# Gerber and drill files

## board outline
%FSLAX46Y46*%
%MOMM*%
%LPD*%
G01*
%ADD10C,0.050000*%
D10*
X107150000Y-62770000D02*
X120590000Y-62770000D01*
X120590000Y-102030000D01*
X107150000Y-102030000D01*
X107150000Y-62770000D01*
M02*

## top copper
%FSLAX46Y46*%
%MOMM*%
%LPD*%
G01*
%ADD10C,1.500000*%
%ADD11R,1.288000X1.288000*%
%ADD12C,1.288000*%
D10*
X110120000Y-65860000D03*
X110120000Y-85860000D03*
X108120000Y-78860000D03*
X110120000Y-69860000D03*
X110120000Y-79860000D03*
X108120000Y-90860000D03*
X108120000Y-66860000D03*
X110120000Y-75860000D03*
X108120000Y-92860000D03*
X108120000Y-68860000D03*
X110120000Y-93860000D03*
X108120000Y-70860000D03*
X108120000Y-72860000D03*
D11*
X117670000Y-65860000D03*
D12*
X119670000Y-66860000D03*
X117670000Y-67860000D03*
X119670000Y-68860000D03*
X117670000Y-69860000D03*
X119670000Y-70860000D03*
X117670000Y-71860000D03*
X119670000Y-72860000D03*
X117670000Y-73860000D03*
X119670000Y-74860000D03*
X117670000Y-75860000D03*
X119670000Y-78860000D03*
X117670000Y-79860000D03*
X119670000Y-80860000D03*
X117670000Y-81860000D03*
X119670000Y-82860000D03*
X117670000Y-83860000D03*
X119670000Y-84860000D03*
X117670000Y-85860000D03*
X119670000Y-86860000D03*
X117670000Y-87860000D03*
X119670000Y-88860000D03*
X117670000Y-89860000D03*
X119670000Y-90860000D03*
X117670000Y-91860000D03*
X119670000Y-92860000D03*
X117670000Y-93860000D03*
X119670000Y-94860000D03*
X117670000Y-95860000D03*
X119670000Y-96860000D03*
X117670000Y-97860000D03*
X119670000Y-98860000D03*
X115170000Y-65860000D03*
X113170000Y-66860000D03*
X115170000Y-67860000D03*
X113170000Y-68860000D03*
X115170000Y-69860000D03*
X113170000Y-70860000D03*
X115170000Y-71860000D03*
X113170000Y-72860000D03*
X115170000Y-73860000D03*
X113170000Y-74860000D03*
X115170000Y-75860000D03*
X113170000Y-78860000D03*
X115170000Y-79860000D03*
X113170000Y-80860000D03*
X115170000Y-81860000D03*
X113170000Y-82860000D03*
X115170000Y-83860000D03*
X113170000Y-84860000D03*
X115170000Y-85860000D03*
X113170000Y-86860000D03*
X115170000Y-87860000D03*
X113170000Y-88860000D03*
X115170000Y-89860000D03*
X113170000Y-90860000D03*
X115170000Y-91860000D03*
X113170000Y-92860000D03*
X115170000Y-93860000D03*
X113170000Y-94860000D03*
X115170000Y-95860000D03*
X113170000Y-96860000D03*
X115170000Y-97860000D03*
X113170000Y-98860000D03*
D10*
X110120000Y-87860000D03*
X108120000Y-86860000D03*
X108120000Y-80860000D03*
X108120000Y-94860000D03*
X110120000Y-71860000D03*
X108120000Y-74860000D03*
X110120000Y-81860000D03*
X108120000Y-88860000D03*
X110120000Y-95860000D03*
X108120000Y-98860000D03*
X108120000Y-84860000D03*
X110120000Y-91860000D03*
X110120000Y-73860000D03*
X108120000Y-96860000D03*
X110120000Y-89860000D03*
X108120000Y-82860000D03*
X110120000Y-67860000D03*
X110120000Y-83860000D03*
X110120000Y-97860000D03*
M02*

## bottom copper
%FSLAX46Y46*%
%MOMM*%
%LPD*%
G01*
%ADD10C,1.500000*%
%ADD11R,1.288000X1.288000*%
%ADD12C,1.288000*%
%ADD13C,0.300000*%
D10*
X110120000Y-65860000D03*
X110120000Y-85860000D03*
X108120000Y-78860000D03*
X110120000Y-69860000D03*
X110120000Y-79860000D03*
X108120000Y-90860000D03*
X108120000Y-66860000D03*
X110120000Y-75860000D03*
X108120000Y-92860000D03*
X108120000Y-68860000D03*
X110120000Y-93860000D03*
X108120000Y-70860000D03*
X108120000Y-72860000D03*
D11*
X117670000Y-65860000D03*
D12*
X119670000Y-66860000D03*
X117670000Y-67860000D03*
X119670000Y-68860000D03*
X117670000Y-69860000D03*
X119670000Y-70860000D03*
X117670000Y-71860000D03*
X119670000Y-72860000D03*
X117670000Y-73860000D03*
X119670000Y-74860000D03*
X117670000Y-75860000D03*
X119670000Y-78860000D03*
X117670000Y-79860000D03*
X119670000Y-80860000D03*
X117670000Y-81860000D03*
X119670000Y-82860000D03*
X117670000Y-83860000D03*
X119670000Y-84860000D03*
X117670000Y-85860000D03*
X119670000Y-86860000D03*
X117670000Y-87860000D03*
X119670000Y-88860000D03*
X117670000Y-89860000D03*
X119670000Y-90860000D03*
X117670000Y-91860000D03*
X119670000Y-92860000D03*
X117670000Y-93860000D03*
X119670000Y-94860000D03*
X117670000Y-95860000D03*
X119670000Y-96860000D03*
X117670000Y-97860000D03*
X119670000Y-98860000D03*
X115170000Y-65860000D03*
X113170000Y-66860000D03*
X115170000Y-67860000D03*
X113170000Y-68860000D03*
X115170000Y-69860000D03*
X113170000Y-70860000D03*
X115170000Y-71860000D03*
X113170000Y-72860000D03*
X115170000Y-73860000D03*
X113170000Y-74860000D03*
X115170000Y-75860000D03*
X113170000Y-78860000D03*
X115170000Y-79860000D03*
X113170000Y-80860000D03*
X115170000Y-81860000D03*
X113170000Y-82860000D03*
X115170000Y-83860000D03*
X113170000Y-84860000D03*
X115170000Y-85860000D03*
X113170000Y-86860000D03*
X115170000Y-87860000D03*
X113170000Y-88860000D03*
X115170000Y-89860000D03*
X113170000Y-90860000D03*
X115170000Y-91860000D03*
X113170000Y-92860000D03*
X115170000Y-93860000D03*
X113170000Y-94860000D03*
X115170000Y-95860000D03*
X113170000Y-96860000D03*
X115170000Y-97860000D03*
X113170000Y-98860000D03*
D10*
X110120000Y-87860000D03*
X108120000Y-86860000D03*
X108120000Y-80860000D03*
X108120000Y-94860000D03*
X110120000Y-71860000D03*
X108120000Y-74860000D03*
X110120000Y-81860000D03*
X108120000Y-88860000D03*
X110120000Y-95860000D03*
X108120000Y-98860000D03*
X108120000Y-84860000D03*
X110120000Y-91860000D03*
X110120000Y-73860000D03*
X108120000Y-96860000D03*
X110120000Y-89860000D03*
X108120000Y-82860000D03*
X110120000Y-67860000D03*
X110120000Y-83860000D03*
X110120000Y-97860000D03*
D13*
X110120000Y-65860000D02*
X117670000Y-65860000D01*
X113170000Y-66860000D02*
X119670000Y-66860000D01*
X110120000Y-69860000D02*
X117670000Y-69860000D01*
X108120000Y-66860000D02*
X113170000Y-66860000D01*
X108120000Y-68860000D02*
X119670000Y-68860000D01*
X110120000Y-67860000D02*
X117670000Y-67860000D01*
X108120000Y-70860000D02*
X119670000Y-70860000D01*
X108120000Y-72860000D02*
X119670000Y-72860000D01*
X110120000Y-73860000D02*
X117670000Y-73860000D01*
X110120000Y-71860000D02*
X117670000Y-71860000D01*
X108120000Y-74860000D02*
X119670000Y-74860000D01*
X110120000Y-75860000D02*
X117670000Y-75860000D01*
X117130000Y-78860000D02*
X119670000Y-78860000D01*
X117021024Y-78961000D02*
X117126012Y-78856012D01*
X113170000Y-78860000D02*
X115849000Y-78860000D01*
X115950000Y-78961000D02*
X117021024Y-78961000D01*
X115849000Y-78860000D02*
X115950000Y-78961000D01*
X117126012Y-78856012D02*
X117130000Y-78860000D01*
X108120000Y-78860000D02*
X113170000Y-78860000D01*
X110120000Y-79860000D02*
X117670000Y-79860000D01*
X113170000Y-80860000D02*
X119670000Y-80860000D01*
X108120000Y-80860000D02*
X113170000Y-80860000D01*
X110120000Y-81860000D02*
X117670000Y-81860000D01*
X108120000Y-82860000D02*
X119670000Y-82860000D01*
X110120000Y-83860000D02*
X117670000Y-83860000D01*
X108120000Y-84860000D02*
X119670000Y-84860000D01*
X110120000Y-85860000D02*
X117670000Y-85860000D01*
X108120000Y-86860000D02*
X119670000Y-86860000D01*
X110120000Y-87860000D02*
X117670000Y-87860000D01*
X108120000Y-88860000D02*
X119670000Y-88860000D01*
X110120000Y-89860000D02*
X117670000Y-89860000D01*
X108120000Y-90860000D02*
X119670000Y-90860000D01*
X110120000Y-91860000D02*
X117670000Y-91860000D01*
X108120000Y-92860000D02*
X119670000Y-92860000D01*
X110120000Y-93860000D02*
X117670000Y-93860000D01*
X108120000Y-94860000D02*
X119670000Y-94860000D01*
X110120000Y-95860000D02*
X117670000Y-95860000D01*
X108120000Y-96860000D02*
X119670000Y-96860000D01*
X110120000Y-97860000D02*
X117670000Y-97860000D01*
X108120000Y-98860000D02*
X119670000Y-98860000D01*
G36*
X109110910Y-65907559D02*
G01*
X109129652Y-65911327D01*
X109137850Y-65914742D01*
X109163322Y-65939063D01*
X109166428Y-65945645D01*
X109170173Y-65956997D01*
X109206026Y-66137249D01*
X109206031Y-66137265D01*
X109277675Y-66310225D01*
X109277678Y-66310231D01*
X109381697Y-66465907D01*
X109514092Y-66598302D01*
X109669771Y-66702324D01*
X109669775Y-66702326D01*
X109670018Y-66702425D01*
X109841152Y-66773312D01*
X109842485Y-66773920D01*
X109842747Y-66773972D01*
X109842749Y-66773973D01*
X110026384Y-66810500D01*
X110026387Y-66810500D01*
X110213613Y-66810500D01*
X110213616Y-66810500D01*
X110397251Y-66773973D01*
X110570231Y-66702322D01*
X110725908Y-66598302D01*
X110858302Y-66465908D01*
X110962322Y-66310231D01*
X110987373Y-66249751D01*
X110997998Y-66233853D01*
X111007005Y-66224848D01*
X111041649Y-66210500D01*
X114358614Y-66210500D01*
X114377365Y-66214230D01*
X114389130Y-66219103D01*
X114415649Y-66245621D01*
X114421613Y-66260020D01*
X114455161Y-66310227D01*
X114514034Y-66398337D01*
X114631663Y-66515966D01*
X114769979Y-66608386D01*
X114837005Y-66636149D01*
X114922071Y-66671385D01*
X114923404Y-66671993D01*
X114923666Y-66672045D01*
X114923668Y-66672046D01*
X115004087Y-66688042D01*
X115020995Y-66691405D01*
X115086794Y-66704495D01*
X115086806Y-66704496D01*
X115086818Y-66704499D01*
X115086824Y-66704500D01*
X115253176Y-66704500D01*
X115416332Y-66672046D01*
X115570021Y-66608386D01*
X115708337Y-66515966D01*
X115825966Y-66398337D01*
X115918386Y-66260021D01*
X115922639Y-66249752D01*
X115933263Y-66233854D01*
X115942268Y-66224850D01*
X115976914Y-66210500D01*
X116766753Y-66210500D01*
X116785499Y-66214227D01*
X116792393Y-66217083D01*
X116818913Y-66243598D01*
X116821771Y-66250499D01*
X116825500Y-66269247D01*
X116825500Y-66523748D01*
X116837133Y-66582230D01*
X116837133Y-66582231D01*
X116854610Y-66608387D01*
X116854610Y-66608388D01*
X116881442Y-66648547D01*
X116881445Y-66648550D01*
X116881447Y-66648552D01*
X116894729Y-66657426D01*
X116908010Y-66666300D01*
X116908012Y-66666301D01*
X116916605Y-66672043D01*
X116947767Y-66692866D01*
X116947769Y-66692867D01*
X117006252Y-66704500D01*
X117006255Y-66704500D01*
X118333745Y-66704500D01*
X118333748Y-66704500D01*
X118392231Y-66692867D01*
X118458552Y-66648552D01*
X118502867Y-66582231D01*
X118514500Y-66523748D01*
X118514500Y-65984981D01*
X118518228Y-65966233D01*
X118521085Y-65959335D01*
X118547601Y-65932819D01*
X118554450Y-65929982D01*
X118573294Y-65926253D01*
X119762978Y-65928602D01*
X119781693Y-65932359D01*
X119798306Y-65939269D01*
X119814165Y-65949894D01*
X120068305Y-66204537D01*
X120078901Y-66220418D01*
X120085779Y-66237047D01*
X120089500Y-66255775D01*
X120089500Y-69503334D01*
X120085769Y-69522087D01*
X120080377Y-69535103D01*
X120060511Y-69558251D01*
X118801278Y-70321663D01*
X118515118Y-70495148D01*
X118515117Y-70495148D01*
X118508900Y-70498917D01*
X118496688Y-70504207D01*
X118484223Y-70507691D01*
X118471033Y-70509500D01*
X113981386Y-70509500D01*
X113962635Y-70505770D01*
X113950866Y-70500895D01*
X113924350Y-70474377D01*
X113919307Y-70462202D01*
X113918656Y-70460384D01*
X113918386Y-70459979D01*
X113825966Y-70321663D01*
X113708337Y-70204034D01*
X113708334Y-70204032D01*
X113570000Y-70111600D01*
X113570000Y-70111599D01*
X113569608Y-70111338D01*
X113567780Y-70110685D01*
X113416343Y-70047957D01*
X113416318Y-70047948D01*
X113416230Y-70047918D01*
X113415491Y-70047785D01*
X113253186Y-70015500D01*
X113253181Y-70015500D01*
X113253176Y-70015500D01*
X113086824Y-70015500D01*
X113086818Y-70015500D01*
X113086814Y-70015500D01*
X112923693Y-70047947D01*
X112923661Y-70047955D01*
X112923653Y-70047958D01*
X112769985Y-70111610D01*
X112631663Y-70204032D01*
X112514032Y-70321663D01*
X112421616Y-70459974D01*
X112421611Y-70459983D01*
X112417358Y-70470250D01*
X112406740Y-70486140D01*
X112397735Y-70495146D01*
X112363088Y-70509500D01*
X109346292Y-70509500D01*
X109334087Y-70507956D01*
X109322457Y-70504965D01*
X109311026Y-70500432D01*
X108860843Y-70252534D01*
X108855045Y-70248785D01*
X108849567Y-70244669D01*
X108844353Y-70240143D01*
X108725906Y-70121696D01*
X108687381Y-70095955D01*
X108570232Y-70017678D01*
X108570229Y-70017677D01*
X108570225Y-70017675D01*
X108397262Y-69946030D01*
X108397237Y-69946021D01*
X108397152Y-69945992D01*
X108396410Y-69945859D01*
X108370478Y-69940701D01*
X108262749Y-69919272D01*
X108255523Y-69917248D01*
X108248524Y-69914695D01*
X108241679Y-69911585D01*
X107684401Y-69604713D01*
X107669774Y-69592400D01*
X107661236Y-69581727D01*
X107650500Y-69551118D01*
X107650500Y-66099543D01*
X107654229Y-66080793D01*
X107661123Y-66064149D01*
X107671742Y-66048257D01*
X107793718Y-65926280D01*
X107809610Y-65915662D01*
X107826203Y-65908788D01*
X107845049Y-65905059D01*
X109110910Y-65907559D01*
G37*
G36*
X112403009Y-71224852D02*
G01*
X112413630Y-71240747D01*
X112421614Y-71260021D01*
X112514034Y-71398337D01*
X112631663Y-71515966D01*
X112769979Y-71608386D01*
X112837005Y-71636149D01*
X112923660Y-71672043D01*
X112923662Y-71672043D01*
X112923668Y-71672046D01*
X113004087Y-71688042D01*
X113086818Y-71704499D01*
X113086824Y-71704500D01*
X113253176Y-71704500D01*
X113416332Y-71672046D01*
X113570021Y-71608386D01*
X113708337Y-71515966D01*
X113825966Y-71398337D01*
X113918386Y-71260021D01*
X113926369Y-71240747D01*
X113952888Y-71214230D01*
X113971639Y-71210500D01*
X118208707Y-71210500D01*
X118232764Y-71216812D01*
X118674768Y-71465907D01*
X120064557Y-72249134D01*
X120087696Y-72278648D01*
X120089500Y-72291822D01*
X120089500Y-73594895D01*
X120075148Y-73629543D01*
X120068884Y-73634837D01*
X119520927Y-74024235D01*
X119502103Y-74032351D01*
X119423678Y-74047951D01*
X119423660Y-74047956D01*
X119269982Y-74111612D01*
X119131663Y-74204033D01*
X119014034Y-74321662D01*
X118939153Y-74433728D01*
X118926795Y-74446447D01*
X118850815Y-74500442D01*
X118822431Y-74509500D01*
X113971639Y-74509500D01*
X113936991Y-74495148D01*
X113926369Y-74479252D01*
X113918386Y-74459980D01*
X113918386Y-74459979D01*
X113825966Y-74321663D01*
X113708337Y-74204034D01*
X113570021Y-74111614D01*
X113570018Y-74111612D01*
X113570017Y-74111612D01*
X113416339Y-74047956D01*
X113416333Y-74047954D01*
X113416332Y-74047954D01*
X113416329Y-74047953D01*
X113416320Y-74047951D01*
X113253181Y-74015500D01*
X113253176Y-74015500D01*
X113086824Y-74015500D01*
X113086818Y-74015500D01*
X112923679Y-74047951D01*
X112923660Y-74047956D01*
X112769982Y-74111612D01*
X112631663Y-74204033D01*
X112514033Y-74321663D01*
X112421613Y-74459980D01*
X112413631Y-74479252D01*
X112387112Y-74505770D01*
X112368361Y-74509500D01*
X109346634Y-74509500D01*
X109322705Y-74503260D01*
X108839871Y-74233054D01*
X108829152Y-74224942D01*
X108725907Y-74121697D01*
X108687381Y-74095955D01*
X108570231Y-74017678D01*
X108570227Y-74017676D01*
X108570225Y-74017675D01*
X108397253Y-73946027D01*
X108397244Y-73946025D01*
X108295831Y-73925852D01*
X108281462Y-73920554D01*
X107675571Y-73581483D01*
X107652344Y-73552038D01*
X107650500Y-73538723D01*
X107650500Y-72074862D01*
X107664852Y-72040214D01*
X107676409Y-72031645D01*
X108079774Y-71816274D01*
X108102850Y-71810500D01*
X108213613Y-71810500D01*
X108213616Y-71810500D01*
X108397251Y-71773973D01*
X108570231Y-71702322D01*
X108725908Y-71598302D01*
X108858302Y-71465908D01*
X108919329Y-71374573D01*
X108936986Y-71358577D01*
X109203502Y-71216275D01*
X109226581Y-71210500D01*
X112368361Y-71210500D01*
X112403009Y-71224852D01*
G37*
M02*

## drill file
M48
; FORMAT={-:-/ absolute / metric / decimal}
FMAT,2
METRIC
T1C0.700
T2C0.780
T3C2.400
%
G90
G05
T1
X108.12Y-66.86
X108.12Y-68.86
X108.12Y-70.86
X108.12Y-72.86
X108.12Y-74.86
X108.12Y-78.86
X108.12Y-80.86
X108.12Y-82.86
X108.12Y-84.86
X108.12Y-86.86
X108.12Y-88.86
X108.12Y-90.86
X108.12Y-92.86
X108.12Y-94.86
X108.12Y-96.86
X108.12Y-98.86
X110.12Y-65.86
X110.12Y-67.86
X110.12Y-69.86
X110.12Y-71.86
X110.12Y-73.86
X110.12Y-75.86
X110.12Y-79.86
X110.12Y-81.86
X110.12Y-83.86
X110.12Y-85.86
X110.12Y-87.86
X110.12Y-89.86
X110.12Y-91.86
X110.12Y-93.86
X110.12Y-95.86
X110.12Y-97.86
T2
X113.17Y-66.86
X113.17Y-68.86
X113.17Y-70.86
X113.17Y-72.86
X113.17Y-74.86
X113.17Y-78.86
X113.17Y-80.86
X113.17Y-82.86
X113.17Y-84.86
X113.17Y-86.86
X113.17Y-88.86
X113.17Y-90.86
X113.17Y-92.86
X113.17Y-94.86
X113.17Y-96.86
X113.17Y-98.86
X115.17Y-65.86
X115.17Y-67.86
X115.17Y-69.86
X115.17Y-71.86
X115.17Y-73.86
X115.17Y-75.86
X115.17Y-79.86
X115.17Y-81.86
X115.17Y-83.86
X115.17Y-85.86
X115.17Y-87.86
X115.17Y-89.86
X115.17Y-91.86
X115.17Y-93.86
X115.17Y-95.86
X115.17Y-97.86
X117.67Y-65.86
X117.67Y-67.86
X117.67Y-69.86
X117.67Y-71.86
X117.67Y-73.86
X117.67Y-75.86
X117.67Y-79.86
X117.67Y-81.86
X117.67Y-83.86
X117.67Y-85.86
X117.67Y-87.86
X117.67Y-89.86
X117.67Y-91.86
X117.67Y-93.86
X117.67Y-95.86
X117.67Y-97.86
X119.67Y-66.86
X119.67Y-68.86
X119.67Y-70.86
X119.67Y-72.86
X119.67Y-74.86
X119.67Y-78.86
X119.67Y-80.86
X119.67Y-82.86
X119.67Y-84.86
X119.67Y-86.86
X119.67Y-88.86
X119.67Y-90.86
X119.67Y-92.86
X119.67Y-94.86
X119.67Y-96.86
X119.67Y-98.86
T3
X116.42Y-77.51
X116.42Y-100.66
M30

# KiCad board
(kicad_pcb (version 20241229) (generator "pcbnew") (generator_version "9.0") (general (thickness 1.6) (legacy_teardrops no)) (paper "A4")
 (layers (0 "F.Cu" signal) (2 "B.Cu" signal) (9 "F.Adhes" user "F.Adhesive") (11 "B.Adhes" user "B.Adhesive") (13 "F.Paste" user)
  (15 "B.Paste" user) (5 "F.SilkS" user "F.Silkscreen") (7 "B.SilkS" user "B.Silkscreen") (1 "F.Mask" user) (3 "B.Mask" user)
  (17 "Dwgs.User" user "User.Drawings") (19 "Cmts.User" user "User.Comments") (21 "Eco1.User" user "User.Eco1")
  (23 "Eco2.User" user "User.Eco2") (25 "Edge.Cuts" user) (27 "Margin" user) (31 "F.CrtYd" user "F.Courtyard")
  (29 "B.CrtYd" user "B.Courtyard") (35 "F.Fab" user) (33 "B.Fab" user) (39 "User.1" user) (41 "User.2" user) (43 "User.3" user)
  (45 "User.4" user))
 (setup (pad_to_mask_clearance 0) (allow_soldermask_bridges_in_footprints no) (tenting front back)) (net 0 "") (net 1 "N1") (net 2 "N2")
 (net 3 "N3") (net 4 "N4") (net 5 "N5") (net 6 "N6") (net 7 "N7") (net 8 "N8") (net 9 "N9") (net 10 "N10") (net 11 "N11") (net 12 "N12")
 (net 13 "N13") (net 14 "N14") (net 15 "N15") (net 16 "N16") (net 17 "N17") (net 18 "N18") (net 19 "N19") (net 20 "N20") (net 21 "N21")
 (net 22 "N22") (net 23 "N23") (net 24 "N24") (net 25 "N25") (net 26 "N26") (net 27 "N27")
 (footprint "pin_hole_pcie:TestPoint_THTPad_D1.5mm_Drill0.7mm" (layer "F.Cu") (at 110.12 65.86 180)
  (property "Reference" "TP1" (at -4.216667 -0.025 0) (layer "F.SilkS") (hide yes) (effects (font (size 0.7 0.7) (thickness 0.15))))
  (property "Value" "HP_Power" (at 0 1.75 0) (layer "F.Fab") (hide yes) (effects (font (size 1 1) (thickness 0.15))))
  (pad "1" thru_hole circle (at 0 0 180) (size 1.5 1.5) (drill 0.7) (layers "*.Cu" "*.Mask") (remove_unused_layers no) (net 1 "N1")))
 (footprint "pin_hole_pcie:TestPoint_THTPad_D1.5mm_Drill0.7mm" (layer "F.Cu") (at 110.12 85.86 180)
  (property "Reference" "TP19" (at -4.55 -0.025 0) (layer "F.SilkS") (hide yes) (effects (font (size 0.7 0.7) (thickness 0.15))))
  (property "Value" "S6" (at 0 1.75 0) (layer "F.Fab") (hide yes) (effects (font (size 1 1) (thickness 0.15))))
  (pad "1" thru_hole circle (at 0 0 180) (size 1.5 1.5) (drill 0.7) (layers "*.Cu" "*.Mask") (remove_unused_layers no) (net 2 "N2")))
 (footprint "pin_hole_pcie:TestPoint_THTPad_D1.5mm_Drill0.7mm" (layer "F.Cu") (at 108.12 78.86 180)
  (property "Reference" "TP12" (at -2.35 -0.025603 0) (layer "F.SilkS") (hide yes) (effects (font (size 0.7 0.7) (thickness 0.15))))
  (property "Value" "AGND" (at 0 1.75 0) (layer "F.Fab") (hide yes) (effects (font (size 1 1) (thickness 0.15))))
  (pad "1" thru_hole circle (at 0 0 180) (size 1.5 1.5) (drill 0.7) (layers "*.Cu" "*.Mask") (remove_unused_layers no) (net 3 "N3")))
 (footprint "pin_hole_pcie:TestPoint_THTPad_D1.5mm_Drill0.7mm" (layer "F.Cu") (at 110.12 69.86 180)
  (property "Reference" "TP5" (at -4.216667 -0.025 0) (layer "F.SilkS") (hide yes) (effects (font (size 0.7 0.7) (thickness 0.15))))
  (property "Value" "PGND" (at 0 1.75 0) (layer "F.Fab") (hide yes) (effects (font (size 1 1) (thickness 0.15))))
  (pad "1" thru_hole circle (at 0 0 180) (size 1.5 1.5) (drill 0.7) (layers "*.Cu" "*.Mask") (remove_unused_layers no) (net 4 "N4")))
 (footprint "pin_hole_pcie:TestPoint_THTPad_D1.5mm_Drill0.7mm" (layer "F.Cu") (at 110.12 79.86 180)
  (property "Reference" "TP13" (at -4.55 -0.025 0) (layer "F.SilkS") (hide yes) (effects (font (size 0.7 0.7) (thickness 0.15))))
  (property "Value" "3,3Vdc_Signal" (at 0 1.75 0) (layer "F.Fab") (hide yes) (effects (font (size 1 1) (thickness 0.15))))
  (pad "1" thru_hole circle (at 0 0 180) (size 1.5 1.5) (drill 0.7) (layers "*.Cu" "*.Mask") (remove_unused_layers no) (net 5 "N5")))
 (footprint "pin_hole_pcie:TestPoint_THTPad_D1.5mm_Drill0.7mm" (layer "F.Cu") (at 108.12 90.86 180)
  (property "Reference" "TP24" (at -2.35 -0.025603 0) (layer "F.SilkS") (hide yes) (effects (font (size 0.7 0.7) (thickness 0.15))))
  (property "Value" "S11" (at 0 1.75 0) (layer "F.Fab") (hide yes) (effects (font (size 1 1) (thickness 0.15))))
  (pad "1" thru_hole circle (at 0 0 180) (size 1.5 1.5) (drill 0.7) (layers "*.Cu" "*.Mask") (remove_unused_layers no) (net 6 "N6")))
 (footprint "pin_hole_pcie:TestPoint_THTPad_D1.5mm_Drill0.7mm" (layer "F.Cu") (at 108.12 66.86 180)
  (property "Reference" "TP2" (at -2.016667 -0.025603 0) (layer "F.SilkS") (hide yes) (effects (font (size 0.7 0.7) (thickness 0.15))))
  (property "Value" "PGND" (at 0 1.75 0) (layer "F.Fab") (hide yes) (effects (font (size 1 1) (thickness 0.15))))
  (pad "1" thru_hole circle (at 0 0 180) (size 1.5 1.5) (drill 0.7) (layers "*.Cu" "*.Mask") (remove_unused_layers no) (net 4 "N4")))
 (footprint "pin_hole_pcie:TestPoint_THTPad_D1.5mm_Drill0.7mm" (layer "F.Cu") (at 110.12 75.86 180)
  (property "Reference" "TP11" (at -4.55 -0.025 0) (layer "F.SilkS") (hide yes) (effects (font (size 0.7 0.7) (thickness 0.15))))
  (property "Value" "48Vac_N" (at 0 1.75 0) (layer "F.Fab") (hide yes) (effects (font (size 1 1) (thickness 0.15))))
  (pad "1" thru_hole circle (at 0 0 180) (size 1.5 1.5) (drill 0.7) (layers "*.Cu" "*.Mask") (remove_unused_layers no) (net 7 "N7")))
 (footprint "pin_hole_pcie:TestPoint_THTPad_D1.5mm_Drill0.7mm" (layer "F.Cu") (at 108.12 92.86 180)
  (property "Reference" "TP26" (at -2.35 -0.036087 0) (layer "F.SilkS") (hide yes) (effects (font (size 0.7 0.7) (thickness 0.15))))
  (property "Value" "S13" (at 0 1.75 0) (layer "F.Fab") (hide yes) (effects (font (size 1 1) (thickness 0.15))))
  (pad "1" thru_hole circle (at 0 0 180) (size 1.5 1.5) (drill 0.7) (layers "*.Cu" "*.Mask") (remove_unused_layers no) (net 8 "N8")))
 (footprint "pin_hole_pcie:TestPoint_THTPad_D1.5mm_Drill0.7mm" (layer "F.Cu") (at 108.12 68.86 180)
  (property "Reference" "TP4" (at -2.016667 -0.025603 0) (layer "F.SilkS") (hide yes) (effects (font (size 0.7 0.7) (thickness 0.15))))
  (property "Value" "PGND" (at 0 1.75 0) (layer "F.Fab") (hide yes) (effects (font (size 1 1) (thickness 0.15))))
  (pad "1" thru_hole circle (at 0 0 180) (size 1.5 1.5) (drill 0.7) (layers "*.Cu" "*.Mask") (remove_unused_layers no) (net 4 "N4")))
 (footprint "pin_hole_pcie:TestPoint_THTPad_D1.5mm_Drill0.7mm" (layer "F.Cu") (at 110.12 93.86 180)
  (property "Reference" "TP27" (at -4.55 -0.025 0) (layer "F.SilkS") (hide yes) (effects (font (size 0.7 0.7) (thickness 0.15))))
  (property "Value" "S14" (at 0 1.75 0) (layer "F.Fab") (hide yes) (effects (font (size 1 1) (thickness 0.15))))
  (pad "1" thru_hole circle (at 0 0 180) (size 1.5 1.5) (drill 0.7) (layers "*.Cu" "*.Mask") (remove_unused_layers no) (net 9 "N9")))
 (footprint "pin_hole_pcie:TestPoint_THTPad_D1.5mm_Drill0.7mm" (layer "F.Cu") (at 108.12 70.86 180)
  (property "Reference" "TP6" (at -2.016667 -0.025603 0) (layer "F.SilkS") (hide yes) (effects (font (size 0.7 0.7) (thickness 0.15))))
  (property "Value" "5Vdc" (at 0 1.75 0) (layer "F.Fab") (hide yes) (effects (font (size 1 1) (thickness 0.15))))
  (pad "1" thru_hole circle (at 0 0 180) (size 1.5 1.5) (drill 0.7) (layers "*.Cu" "*.Mask") (remove_unused_layers no) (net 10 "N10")))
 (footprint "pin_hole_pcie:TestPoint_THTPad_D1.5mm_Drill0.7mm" (layer "F.Cu") (at 108.12 72.86 180)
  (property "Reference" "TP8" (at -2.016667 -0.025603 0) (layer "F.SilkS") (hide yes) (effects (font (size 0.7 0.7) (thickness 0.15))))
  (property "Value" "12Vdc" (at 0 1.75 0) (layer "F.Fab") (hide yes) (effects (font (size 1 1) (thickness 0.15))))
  (pad "1" thru_hole circle (at 0 0 180) (size 1.5 1.5) (drill 0.7) (layers "*.Cu" "*.Mask") (remove_unused_layers no) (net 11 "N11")))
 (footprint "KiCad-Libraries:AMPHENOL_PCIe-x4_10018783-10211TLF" (layer "F.Cu") (at 116.42 77.51 -90)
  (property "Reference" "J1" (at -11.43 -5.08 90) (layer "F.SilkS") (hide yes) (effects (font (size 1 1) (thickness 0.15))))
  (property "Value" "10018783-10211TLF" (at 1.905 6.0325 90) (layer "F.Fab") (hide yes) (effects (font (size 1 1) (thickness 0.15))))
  (pad "" np_thru_hole circle (at 0 0 270) (size 2.4 2.4) (drill 2.4) (layers "*.Cu" "*.Mask"))
  (pad "" np_thru_hole circle (at 23.15 0 270) (size 2.4 2.4) (drill 2.4) (layers "*.Cu" "*.Mask"))
  (pad "A1" thru_hole rect (at -11.65 -1.25 270) (size 1.288 1.288) (drill 0.78) (layers "*.Cu" "*.Mask") (remove_unused_layers no)
   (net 1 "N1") (solder_mask_margin 0.102))
  (pad "A2" thru_hole circle (at -10.65 -3.25 270) (size 1.288 1.288) (drill 0.78) (layers "*.Cu" "*.Mask") (remove_unused_layers no)
   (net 4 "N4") (solder_mask_margin 0.102))
  (pad "A3" thru_hole circle (at -9.65 -1.25 270) (size 1.288 1.288) (drill 0.78) (layers "*.Cu" "*.Mask") (remove_unused_layers no)
   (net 4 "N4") (solder_mask_margin 0.102))
  (pad "A4" thru_hole circle (at -8.65 -3.25 270) (size 1.288 1.288) (drill 0.78) (layers "*.Cu" "*.Mask") (remove_unused_layers no)
   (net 4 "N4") (solder_mask_margin 0.102))
  (pad "A5" thru_hole circle (at -7.65 -1.25 270) (size 1.288 1.288) (drill 0.78) (layers "*.Cu" "*.Mask") (remove_unused_layers no)
   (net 4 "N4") (solder_mask_margin 0.102))
  (pad "A6" thru_hole circle (at -6.65 -3.25 270) (size 1.288 1.288) (drill 0.78) (layers "*.Cu" "*.Mask") (remove_unused_layers no)
   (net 10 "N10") (solder_mask_margin 0.102))
  (pad "A7" thru_hole circle (at -5.65 -1.25 270) (size 1.288 1.288) (drill 0.78) (layers "*.Cu" "*.Mask") (remove_unused_layers no)
   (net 11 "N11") (solder_mask_margin 0.102))
  (pad "A8" thru_hole circle (at -4.65 -3.25 270) (size 1.288 1.288) (drill 0.78) (layers "*.Cu" "*.Mask") (remove_unused_layers no)
   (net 11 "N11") (solder_mask_margin 0.102))
  (pad "A9" thru_hole circle (at -3.65 -1.25 270) (size 1.288 1.288) (drill 0.78) (layers "*.Cu" "*.Mask") (remove_unused_layers no)
   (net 11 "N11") (solder_mask_margin 0.102))
  (pad "A10" thru_hole circle (at -2.65 -3.25 270) (size 1.288 1.288) (drill 0.78) (layers "*.Cu" "*.Mask") (remove_unused_layers no)
   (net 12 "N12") (solder_mask_margin 0.102))
  (pad "A11" thru_hole circle (at -1.65 -1.25 270) (size 1.288 1.288) (drill 0.78) (layers "*.Cu" "*.Mask") (remove_unused_layers no)
   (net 7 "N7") (solder_mask_margin 0.102))
  (pad "A12" thru_hole circle (at 1.35 -3.25 270) (size 1.288 1.288) (drill 0.78) (layers "*.Cu" "*.Mask") (remove_unused_layers no)
   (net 3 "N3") (solder_mask_margin 0.102))
  (pad "A13" thru_hole circle (at 2.35 -1.25 270) (size 1.288 1.288) (drill 0.78) (layers "*.Cu" "*.Mask") (remove_unused_layers no)
   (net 5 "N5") (solder_mask_margin 0.102))
  (pad "A14" thru_hole circle (at 3.35 -3.25 270) (size 1.288 1.288) (drill 0.78) (layers "*.Cu" "*.Mask") (remove_unused_layers no)
   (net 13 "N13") (solder_mask_margin 0.102))
  (pad "A15" thru_hole circle (at 4.35 -1.25 270) (size 1.288 1.288) (drill 0.78) (layers "*.Cu" "*.Mask") (remove_unused_layers no)
   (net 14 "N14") (solder_mask_margin 0.102))
  (pad "A16" thru_hole circle (at 5.35 -3.25 270) (size 1.288 1.288) (drill 0.78) (layers "*.Cu" "*.Mask") (remove_unused_layers no)
   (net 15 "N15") (solder_mask_margin 0.102))
  (pad "A17" thru_hole circle (at 6.35 -1.25 270) (size 1.288 1.288) (drill 0.78) (layers "*.Cu" "*.Mask") (remove_unused_layers no)
   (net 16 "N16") (solder_mask_margin 0.102))
  (pad "A18" thru_hole circle (at 7.35 -3.25 270) (size 1.288 1.288) (drill 0.78) (layers "*.Cu" "*.Mask") (remove_unused_layers no)
   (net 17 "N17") (solder_mask_margin 0.102))
  (pad "A19" thru_hole circle (at 8.35 -1.25 270) (size 1.288 1.288) (drill 0.78) (layers "*.Cu" "*.Mask") (remove_unused_layers no)
   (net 2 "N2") (solder_mask_margin 0.102))
  (pad "A20" thru_hole circle (at 9.35 -3.25 270) (size 1.288 1.288) (drill 0.78) (layers "*.Cu" "*.Mask") (remove_unused_layers no)
   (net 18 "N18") (solder_mask_margin 0.102))
  (pad "A21" thru_hole circle (at 10.35 -1.25 270) (size 1.288 1.288) (drill 0.78) (layers "*.Cu" "*.Mask") (remove_unused_layers no)
   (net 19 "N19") (solder_mask_margin 0.102))
  (pad "A22" thru_hole circle (at 11.35 -3.25 270) (size 1.288 1.288) (drill 0.78) (layers "*.Cu" "*.Mask") (remove_unused_layers no)
   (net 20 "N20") (solder_mask_margin 0.102))
  (pad "A23" thru_hole circle (at 12.35 -1.25 270) (size 1.288 1.288) (drill 0.78) (layers "*.Cu" "*.Mask") (remove_unused_layers no)
   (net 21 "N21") (solder_mask_margin 0.102))
  (pad "A24" thru_hole circle (at 13.35 -3.25 270) (size 1.288 1.288) (drill 0.78) (layers "*.Cu" "*.Mask") (remove_unused_layers no)
   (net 6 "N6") (solder_mask_margin 0.102))
  (pad "A25" thru_hole circle (at 14.35 -1.25 270) (size 1.288 1.288) (drill 0.78) (layers "*.Cu" "*.Mask") (remove_unused_layers no)
   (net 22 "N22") (solder_mask_margin 0.102))
  (pad "A26" thru_hole circle (at 15.35 -3.25 270) (size 1.288 1.288) (drill 0.78) (layers "*.Cu" "*.Mask") (remove_unused_layers no)
   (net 8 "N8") (solder_mask_margin 0.102))
  (pad "A27" thru_hole circle (at 16.35 -1.25 270) (size 1.288 1.288) (drill 0.78) (layers "*.Cu" "*.Mask") (remove_unused_layers no)
   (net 9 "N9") (solder_mask_margin 0.102))
  (pad "A28" thru_hole circle (at 17.35 -3.25 270) (size 1.288 1.288) (drill 0.78) (layers "*.Cu" "*.Mask") (remove_unused_layers no)
   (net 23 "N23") (solder_mask_margin 0.102))
  (pad "A29" thru_hole circle (at 18.35 -1.25 270) (size 1.288 1.288) (drill 0.78) (layers "*.Cu" "*.Mask") (remove_unused_layers no)
   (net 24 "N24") (solder_mask_margin 0.102))
  (pad "A30" thru_hole circle (at 19.35 -3.25 270) (size 1.288 1.288) (drill 0.78) (layers "*.Cu" "*.Mask") (remove_unused_layers no)
   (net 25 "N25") (solder_mask_margin 0.102))
  (pad "A31" thru_hole circle (at 20.35 -1.25 270) (size 1.288 1.288) (drill 0.78) (layers "*.Cu" "*.Mask") (remove_unused_layers no)
   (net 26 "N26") (solder_mask_margin 0.102))
  (pad "A32" thru_hole circle (at 21.35 -3.25 270) (size 1.288 1.288) (drill 0.78) (layers "*.Cu" "*.Mask") (remove_unused_layers no)
   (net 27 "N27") (solder_mask_margin 0.102))
  (pad "B1" thru_hole circle (at -11.65 1.25 270) (size 1.288 1.288) (drill 0.78) (layers "*.Cu" "*.Mask") (remove_unused_layers no)
   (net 1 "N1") (solder_mask_margin 0.102))
  (pad "B2" thru_hole circle (at -10.65 3.25 270) (size 1.288 1.288) (drill 0.78) (layers "*.Cu" "*.Mask") (remove_unused_layers no)
   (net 4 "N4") (solder_mask_margin 0.102))
  (pad "B3" thru_hole circle (at -9.65 1.25 270) (size 1.288 1.288) (drill 0.78) (layers "*.Cu" "*.Mask") (remove_unused_layers no)
   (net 4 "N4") (solder_mask_margin 0.102))
  (pad "B4" thru_hole circle (at -8.65 3.25 270) (size 1.288 1.288) (drill 0.78) (layers "*.Cu" "*.Mask") (remove_unused_layers no)
   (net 4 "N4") (solder_mask_margin 0.102))
  (pad "B5" thru_hole circle (at -7.65 1.25 270) (size 1.288 1.288) (drill 0.78) (layers "*.Cu" "*.Mask") (remove_unused_layers no)
   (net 4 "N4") (solder_mask_margin 0.102))
  (pad "B6" thru_hole circle (at -6.65 3.25 270) (size 1.288 1.288) (drill 0.78) (layers "*.Cu" "*.Mask") (remove_unused_layers no)
   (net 10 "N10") (solder_mask_margin 0.102))
  (pad "B7" thru_hole circle (at -5.65 1.25 270) (size 1.288 1.288) (drill 0.78) (layers "*.Cu" "*.Mask") (remove_unused_layers no)
   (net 11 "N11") (solder_mask_margin 0.102))
  (pad "B8" thru_hole circle (at -4.65 3.25 270) (size 1.288 1.288) (drill 0.78) (layers "*.Cu" "*.Mask") (remove_unused_layers no)
   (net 11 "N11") (solder_mask_margin 0.102))
  (pad "B9" thru_hole circle (at -3.65 1.25 270) (size 1.288 1.288) (drill 0.78) (layers "*.Cu" "*.Mask") (remove_unused_layers no)
   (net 11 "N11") (solder_mask_margin 0.102))
  (pad "B10" thru_hole circle (at -2.65 3.25 270) (size 1.288 1.288) (drill 0.78) (layers "*.Cu" "*.Mask") (remove_unused_layers no)
   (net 12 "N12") (solder_mask_margin 0.102))
  (pad "B11" thru_hole circle (at -1.65 1.25 270) (size 1.288 1.288) (drill 0.78) (layers "*.Cu" "*.Mask") (remove_unused_layers no)
   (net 7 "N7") (solder_mask_margin 0.102))
  (pad "B12" thru_hole circle (at 1.35 3.25 270) (size 1.288 1.288) (drill 0.78) (layers "*.Cu" "*.Mask") (remove_unused_layers no)
   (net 3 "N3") (solder_mask_margin 0.102))
  (pad "B13" thru_hole circle (at 2.35 1.25 270) (size 1.288 1.288) (drill 0.78) (layers "*.Cu" "*.Mask") (remove_unused_layers no)
   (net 5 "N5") (solder_mask_margin 0.102))
  (pad "B14" thru_hole circle (at 3.35 3.25 270) (size 1.288 1.288) (drill 0.78) (layers "*.Cu" "*.Mask") (remove_unused_layers no)
   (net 13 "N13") (solder_mask_margin 0.102))
  (pad "B15" thru_hole circle (at 4.35 1.25 270) (size 1.288 1.288) (drill 0.78) (layers "*.Cu" "*.Mask") (remove_unused_layers no)
   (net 14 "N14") (solder_mask_margin 0.102))
  (pad "B16" thru_hole circle (at 5.35 3.25 270) (size 1.288 1.288) (drill 0.78) (layers "*.Cu" "*.Mask") (remove_unused_layers no)
   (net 15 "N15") (solder_mask_margin 0.102))
  (pad "B17" thru_hole circle (at 6.35 1.25 270) (size 1.288 1.288) (drill 0.78) (layers "*.Cu" "*.Mask") (remove_unused_layers no)
   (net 16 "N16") (solder_mask_margin 0.102))
  (pad "B18" thru_hole circle (at 7.35 3.25 270) (size 1.288 1.288) (drill 0.78) (layers "*.Cu" "*.Mask") (remove_unused_layers no)
   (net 17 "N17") (solder_mask_margin 0.102))
  (pad "B19" thru_hole circle (at 8.35 1.25 270) (size 1.288 1.288) (drill 0.78) (layers "*.Cu" "*.Mask") (remove_unused_layers no)
   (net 2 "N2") (solder_mask_margin 0.102))
  (pad "B20" thru_hole circle (at 9.35 3.25 270) (size 1.288 1.288) (drill 0.78) (layers "*.Cu" "*.Mask") (remove_unused_layers no)
   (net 18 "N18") (solder_mask_margin 0.102))
  (pad "B21" thru_hole circle (at 10.35 1.25 270) (size 1.288 1.288) (drill 0.78) (layers "*.Cu" "*.Mask") (remove_unused_layers no)
   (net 19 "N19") (solder_mask_margin 0.102))
  (pad "B22" thru_hole circle (at 11.35 3.25 270) (size 1.288 1.288) (drill 0.78) (layers "*.Cu" "*.Mask") (remove_unused_layers no)
   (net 20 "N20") (solder_mask_margin 0.102))
  (pad "B23" thru_hole circle (at 12.35 1.25 270) (size 1.288 1.288) (drill 0.78) (layers "*.Cu" "*.Mask") (remove_unused_layers no)
   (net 21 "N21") (solder_mask_margin 0.102))
  (pad "B24" thru_hole circle (at 13.35 3.25 270) (size 1.288 1.288) (drill 0.78) (layers "*.Cu" "*.Mask") (remove_unused_layers no)
   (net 6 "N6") (solder_mask_margin 0.102))
  (pad "B25" thru_hole circle (at 14.35 1.25 270) (size 1.288 1.288) (drill 0.78) (layers "*.Cu" "*.Mask") (remove_unused_layers no)
   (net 22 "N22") (solder_mask_margin 0.102))
  (pad "B26" thru_hole circle (at 15.35 3.25 270) (size 1.288 1.288) (drill 0.78) (layers "*.Cu" "*.Mask") (remove_unused_layers no)
   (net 8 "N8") (solder_mask_margin 0.102))
  (pad "B27" thru_hole circle (at 16.35 1.25 270) (size 1.288 1.288) (drill 0.78) (layers "*.Cu" "*.Mask") (remove_unused_layers no)
   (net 9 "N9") (solder_mask_margin 0.102))
  (pad "B28" thru_hole circle (at 17.35 3.25 270) (size 1.288 1.288) (drill 0.78) (layers "*.Cu" "*.Mask") (remove_unused_layers no)
   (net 23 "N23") (solder_mask_margin 0.102))
  (pad "B29" thru_hole circle (at 18.35 1.25 270) (size 1.288 1.288) (drill 0.78) (layers "*.Cu" "*.Mask") (remove_unused_layers no)
   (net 24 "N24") (solder_mask_margin 0.102))
  (pad "B30" thru_hole circle (at 19.35 3.25 270) (size 1.288 1.288) (drill 0.78) (layers "*.Cu" "*.Mask") (remove_unused_layers no)
   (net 25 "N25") (solder_mask_margin 0.102))
  (pad "B31" thru_hole circle (at 20.35 1.25 270) (size 1.288 1.288) (drill 0.78) (layers "*.Cu" "*.Mask") (remove_unused_layers no)
   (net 26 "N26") (solder_mask_margin 0.102))
  (pad "B32" thru_hole circle (at 21.35 3.25 270) (size 1.288 1.288) (drill 0.78) (layers "*.Cu" "*.Mask") (remove_unused_layers no)
   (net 27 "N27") (solder_mask_margin 0.102)))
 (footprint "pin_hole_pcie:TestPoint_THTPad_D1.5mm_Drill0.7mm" (layer "F.Cu") (at 110.12 87.86 180)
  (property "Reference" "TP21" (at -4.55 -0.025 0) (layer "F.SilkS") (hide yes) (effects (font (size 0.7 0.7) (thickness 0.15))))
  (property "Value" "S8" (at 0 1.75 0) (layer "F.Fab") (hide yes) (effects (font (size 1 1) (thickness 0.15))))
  (pad "1" thru_hole circle (at 0 0 180) (size 1.5 1.5) (drill 0.7) (layers "*.Cu" "*.Mask") (remove_unused_layers no) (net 19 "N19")))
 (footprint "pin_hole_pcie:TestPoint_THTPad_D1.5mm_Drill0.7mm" (layer "F.Cu") (at 108.12 86.86 180)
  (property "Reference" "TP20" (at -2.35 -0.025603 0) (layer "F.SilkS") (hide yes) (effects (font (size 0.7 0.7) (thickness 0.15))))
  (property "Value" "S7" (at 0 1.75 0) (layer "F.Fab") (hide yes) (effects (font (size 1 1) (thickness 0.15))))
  (pad "1" thru_hole circle (at 0 0 180) (size 1.5 1.5) (drill 0.7) (layers "*.Cu" "*.Mask") (remove_unused_layers no) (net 18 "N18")))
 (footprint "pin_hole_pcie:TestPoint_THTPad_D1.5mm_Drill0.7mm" (layer "F.Cu") (at 108.12 80.86 180)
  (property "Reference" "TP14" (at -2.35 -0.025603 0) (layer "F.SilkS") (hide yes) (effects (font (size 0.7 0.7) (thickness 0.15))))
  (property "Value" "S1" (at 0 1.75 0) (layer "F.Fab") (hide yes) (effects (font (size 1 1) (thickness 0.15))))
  (pad "1" thru_hole circle (at 0 0 180) (size 1.5 1.5) (drill 0.7) (layers "*.Cu" "*.Mask") (remove_unused_layers no) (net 13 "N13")))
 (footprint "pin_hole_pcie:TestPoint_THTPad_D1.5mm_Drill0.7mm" (layer "F.Cu") (at 108.12 94.86 180)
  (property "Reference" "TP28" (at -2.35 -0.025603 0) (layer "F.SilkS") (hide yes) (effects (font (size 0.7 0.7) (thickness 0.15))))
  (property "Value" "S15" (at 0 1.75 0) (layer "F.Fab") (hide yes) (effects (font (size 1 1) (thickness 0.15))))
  (pad "1" thru_hole circle (at 0 0 180) (size 1.5 1.5) (drill 0.7) (layers "*.Cu" "*.Mask") (remove_unused_layers no) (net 23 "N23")))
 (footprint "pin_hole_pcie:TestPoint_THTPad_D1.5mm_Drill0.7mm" (layer "F.Cu") (at 110.12 71.86 180)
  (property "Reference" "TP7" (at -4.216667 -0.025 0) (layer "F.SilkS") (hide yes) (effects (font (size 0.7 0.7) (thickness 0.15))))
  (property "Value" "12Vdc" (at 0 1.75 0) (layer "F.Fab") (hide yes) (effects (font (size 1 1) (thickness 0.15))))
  (pad "1" thru_hole circle (at 0 0 180) (size 1.5 1.5) (drill 0.7) (layers "*.Cu" "*.Mask") (remove_unused_layers no) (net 11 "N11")))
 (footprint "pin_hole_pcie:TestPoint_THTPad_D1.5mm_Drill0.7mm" (layer "F.Cu") (at 108.12 74.86 180)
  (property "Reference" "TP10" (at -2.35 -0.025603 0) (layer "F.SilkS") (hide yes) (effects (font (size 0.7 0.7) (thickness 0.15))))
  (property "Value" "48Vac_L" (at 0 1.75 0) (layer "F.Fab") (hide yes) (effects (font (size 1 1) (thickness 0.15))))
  (pad "1" thru_hole circle (at 0 0 180) (size 1.5 1.5) (drill 0.7) (layers "*.Cu" "*.Mask") (remove_unused_layers no) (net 12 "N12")))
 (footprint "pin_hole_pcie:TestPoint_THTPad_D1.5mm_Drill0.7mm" (layer "F.Cu") (at 110.12 81.86 180)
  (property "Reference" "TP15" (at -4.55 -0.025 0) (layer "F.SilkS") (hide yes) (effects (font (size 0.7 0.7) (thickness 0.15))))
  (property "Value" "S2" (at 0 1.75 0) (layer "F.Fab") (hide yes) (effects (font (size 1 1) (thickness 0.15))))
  (pad "1" thru_hole circle (at 0 0 180) (size 1.5 1.5) (drill 0.7) (layers "*.Cu" "*.Mask") (remove_unused_layers no) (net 14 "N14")))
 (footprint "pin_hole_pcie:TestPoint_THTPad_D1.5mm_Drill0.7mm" (layer "F.Cu") (at 108.12 88.86 180)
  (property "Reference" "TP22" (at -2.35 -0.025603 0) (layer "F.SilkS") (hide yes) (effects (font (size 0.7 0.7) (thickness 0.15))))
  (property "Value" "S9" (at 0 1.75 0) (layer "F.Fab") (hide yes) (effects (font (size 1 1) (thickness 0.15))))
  (pad "1" thru_hole circle (at 0 0 180) (size 1.5 1.5) (drill 0.7) (layers "*.Cu" "*.Mask") (remove_unused_layers no) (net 20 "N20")))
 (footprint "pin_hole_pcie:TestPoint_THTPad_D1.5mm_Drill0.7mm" (layer "F.Cu") (at 110.12 95.86 180)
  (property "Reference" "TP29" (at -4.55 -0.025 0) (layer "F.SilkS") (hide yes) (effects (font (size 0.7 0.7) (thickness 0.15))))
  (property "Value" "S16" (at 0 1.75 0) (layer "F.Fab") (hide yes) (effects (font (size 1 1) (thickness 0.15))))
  (pad "1" thru_hole circle (at 0 0 180) (size 1.5 1.5) (drill 0.7) (layers "*.Cu" "*.Mask") (remove_unused_layers no) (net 24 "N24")))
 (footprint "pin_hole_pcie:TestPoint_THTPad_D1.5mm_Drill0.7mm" (layer "F.Cu") (at 108.12 98.86 180)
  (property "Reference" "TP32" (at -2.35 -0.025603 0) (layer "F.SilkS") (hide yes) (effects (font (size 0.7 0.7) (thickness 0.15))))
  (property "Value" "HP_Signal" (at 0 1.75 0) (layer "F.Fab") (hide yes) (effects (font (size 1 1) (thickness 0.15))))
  (pad "1" thru_hole circle (at 0 0 180) (size 1.5 1.5) (drill 0.7) (layers "*.Cu" "*.Mask") (remove_unused_layers no) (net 27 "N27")))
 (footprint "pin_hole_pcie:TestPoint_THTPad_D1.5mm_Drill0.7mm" (layer "F.Cu") (at 108.12 84.86 180)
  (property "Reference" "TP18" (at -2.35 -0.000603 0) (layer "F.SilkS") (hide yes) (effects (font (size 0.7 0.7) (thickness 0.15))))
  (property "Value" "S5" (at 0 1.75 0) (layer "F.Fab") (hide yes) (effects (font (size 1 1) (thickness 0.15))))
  (pad "1" thru_hole circle (at 0 0 180) (size 1.5 1.5) (drill 0.7) (layers "*.Cu" "*.Mask") (remove_unused_layers no) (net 17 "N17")))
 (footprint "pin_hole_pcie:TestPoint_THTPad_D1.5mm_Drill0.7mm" (layer "F.Cu") (at 110.12 91.86 180)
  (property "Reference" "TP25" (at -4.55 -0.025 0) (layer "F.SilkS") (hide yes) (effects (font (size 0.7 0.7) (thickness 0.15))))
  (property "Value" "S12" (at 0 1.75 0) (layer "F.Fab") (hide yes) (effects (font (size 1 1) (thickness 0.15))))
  (pad "1" thru_hole circle (at 0 0 180) (size 1.5 1.5) (drill 0.7) (layers "*.Cu" "*.Mask") (remove_unused_layers no) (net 22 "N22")))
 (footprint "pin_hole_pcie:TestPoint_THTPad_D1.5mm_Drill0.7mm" (layer "F.Cu") (at 110.12 73.86 180)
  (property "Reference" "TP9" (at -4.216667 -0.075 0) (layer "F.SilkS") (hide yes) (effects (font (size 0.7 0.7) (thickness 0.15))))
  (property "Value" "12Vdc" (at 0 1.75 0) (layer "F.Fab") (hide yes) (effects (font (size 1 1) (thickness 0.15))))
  (pad "1" thru_hole circle (at 0 0 180) (size 1.5 1.5) (drill 0.7) (layers "*.Cu" "*.Mask") (remove_unused_layers no) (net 11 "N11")))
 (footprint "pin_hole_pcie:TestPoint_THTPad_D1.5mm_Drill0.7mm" (layer "F.Cu") (at 108.12 96.86 180)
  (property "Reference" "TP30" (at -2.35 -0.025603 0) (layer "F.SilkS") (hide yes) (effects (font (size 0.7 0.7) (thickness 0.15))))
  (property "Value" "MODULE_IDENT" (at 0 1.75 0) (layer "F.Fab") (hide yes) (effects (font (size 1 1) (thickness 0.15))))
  (pad "1" thru_hole circle (at 0 0 180) (size 1.5 1.5) (drill 0.7) (layers "*.Cu" "*.Mask") (remove_unused_layers no) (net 25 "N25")))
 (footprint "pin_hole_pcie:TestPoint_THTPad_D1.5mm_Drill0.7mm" (layer "F.Cu") (at 110.12 89.86 180)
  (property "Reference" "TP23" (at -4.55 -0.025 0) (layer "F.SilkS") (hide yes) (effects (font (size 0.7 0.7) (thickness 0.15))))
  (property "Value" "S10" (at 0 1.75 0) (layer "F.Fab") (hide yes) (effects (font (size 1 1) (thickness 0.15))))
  (pad "1" thru_hole circle (at 0 0 180) (size 1.5 1.5) (drill 0.7) (layers "*.Cu" "*.Mask") (remove_unused_layers no) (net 21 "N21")))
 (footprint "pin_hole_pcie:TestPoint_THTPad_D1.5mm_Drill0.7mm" (layer "F.Cu") (at 108.12 82.86 180)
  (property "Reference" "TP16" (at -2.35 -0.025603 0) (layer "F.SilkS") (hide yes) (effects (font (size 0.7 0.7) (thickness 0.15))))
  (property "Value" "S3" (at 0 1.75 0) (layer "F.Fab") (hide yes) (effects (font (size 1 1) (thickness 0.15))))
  (pad "1" thru_hole circle (at 0 0 180) (size 1.5 1.5) (drill 0.7) (layers "*.Cu" "*.Mask") (remove_unused_layers no) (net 15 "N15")))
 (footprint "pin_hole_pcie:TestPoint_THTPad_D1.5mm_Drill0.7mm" (layer "F.Cu") (at 110.12 67.86 180)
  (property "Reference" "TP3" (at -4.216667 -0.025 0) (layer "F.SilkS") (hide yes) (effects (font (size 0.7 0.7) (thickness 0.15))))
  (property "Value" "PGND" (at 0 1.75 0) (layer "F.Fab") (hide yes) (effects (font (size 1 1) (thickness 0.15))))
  (pad "1" thru_hole circle (at 0 0 180) (size 1.5 1.5) (drill 0.7) (layers "*.Cu" "*.Mask") (remove_unused_layers no) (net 4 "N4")))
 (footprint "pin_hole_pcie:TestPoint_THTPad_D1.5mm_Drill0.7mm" (layer "F.Cu") (at 110.12 83.86 180)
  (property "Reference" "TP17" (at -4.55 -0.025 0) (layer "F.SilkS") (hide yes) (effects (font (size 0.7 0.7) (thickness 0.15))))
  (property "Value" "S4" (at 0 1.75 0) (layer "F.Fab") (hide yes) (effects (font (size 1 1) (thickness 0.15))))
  (pad "1" thru_hole circle (at 0 0 180) (size 1.5 1.5) (drill 0.7) (layers "*.Cu" "*.Mask") (remove_unused_layers no) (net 16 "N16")))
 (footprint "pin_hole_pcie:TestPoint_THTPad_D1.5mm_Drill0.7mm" (layer "F.Cu") (at 110.12 97.86 180)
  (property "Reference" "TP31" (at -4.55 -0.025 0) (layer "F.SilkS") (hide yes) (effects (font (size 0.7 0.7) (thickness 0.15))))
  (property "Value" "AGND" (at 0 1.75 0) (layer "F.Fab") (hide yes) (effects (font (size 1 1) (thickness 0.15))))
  (pad "1" thru_hole circle (at 0 0 180) (size 1.5 1.5) (drill 0.7) (layers "*.Cu" "*.Mask") (remove_unused_layers no) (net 26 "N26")))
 (gr_rect (start 107.15 62.77) (end 120.59 102.03) (stroke (width 0.05) (type default)) (fill no) (layer "Edge.Cuts"))
 (segment (start 110.12 65.86) (end 117.67 65.86) (width 0.3) (layer "B.Cu") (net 1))
 (segment (start 113.17 66.86) (end 119.67 66.86) (width 0.3) (layer "B.Cu") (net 4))
 (segment (start 110.12 69.86) (end 117.67 69.86) (width 0.3) (layer "B.Cu") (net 4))
 (segment (start 108.12 66.86) (end 113.17 66.86) (width 0.3) (layer "B.Cu") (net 4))
 (segment (start 108.12 68.86) (end 119.67 68.86) (width 0.3) (layer "B.Cu") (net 4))
 (segment (start 110.12 67.86) (end 117.67 67.86) (width 0.3) (layer "B.Cu") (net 4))
 (segment (start 108.12 70.86) (end 119.67 70.86) (width 0.3) (layer "B.Cu") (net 10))
 (segment (start 108.12 72.86) (end 119.67 72.86) (width 0.3) (layer "B.Cu") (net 11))
 (segment (start 110.12 73.86) (end 117.67 73.86) (width 0.3) (layer "B.Cu") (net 11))
 (segment (start 110.12 71.86) (end 117.67 71.86) (width 0.3) (layer "B.Cu") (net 11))
 (segment (start 108.12 74.86) (end 119.67 74.86) (width 0.3) (layer "B.Cu") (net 12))
 (segment (start 110.12 75.86) (end 117.67 75.86) (width 0.3) (layer "B.Cu") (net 7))
 (segment (start 117.13 78.86) (end 119.67 78.86) (width 0.3) (layer "B.Cu") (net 3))
 (segment (start 117.021024 78.961) (end 117.126012 78.856012) (width 0.3) (layer "B.Cu") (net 3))
 (segment (start 113.17 78.86) (end 115.849 78.86) (width 0.3) (layer "B.Cu") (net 3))
 (segment (start 115.95 78.961) (end 117.021024 78.961) (width 0.3) (layer "B.Cu") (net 3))
 (segment (start 115.849 78.86) (end 115.95 78.961) (width 0.3) (layer "B.Cu") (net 3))
 (segment (start 117.126012 78.856012) (end 117.13 78.86) (width 0.3) (layer "B.Cu") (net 3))
 (segment (start 108.12 78.86) (end 113.17 78.86) (width 0.3) (layer "B.Cu") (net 3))
 (segment (start 110.12 79.86) (end 117.67 79.86) (width 0.3) (layer "B.Cu") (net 5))
 (segment (start 113.17 80.86) (end 119.67 80.86) (width 0.3) (layer "B.Cu") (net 13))
 (segment (start 108.12 80.86) (end 113.17 80.86) (width 0.3) (layer "B.Cu") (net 13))
 (segment (start 110.12 81.86) (end 117.67 81.86) (width 0.3) (layer "B.Cu") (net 14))
 (segment (start 108.12 82.86) (end 119.67 82.86) (width 0.3) (layer "B.Cu") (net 15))
 (segment (start 110.12 83.86) (end 117.67 83.86) (width 0.3) (layer "B.Cu") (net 16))
 (segment (start 108.12 84.86) (end 119.67 84.86) (width 0.3) (layer "B.Cu") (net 17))
 (segment (start 110.12 85.86) (end 117.67 85.86) (width 0.3) (layer "B.Cu") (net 2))
 (segment (start 108.12 86.86) (end 119.67 86.86) (width 0.3) (layer "B.Cu") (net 18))
 (segment (start 110.12 87.86) (end 117.67 87.86) (width 0.3) (layer "B.Cu") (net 19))
 (segment (start 108.12 88.86) (end 119.67 88.86) (width 0.3) (layer "B.Cu") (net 20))
 (segment (start 110.12 89.86) (end 117.67 89.86) (width 0.3) (layer "B.Cu") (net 21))
 (segment (start 108.12 90.86) (end 119.67 90.86) (width 0.3) (layer "B.Cu") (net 6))
 (segment (start 110.12 91.86) (end 117.67 91.86) (width 0.3) (layer "B.Cu") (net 22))
 (segment (start 108.12 92.86) (end 119.67 92.86) (width 0.3) (layer "B.Cu") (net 8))
 (segment (start 110.12 93.86) (end 117.67 93.86) (width 0.3) (layer "B.Cu") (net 9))
 (segment (start 108.12 94.86) (end 119.67 94.86) (width 0.3) (layer "B.Cu") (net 23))
 (segment (start 110.12 95.86) (end 117.67 95.86) (width 0.3) (layer "B.Cu") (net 24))
 (segment (start 108.12 96.86) (end 119.67 96.86) (width 0.3) (layer "B.Cu") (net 25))
 (segment (start 110.12 97.86) (end 117.67 97.86) (width 0.3) (layer "B.Cu") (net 26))
 (segment (start 108.12 98.86) (end 119.67 98.86) (width 0.3) (layer "B.Cu") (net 27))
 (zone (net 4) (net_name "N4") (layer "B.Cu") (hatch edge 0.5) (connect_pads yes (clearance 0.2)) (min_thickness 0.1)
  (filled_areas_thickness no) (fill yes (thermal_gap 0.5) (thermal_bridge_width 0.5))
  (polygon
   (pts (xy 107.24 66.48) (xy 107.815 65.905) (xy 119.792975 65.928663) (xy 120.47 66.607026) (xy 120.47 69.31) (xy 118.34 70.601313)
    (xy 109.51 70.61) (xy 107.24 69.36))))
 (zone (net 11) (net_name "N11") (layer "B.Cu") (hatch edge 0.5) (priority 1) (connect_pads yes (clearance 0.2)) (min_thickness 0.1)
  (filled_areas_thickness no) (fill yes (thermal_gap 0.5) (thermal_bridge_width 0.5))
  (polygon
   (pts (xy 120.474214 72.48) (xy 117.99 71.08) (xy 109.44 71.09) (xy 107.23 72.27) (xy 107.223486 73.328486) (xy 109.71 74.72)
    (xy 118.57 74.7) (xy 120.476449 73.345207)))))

